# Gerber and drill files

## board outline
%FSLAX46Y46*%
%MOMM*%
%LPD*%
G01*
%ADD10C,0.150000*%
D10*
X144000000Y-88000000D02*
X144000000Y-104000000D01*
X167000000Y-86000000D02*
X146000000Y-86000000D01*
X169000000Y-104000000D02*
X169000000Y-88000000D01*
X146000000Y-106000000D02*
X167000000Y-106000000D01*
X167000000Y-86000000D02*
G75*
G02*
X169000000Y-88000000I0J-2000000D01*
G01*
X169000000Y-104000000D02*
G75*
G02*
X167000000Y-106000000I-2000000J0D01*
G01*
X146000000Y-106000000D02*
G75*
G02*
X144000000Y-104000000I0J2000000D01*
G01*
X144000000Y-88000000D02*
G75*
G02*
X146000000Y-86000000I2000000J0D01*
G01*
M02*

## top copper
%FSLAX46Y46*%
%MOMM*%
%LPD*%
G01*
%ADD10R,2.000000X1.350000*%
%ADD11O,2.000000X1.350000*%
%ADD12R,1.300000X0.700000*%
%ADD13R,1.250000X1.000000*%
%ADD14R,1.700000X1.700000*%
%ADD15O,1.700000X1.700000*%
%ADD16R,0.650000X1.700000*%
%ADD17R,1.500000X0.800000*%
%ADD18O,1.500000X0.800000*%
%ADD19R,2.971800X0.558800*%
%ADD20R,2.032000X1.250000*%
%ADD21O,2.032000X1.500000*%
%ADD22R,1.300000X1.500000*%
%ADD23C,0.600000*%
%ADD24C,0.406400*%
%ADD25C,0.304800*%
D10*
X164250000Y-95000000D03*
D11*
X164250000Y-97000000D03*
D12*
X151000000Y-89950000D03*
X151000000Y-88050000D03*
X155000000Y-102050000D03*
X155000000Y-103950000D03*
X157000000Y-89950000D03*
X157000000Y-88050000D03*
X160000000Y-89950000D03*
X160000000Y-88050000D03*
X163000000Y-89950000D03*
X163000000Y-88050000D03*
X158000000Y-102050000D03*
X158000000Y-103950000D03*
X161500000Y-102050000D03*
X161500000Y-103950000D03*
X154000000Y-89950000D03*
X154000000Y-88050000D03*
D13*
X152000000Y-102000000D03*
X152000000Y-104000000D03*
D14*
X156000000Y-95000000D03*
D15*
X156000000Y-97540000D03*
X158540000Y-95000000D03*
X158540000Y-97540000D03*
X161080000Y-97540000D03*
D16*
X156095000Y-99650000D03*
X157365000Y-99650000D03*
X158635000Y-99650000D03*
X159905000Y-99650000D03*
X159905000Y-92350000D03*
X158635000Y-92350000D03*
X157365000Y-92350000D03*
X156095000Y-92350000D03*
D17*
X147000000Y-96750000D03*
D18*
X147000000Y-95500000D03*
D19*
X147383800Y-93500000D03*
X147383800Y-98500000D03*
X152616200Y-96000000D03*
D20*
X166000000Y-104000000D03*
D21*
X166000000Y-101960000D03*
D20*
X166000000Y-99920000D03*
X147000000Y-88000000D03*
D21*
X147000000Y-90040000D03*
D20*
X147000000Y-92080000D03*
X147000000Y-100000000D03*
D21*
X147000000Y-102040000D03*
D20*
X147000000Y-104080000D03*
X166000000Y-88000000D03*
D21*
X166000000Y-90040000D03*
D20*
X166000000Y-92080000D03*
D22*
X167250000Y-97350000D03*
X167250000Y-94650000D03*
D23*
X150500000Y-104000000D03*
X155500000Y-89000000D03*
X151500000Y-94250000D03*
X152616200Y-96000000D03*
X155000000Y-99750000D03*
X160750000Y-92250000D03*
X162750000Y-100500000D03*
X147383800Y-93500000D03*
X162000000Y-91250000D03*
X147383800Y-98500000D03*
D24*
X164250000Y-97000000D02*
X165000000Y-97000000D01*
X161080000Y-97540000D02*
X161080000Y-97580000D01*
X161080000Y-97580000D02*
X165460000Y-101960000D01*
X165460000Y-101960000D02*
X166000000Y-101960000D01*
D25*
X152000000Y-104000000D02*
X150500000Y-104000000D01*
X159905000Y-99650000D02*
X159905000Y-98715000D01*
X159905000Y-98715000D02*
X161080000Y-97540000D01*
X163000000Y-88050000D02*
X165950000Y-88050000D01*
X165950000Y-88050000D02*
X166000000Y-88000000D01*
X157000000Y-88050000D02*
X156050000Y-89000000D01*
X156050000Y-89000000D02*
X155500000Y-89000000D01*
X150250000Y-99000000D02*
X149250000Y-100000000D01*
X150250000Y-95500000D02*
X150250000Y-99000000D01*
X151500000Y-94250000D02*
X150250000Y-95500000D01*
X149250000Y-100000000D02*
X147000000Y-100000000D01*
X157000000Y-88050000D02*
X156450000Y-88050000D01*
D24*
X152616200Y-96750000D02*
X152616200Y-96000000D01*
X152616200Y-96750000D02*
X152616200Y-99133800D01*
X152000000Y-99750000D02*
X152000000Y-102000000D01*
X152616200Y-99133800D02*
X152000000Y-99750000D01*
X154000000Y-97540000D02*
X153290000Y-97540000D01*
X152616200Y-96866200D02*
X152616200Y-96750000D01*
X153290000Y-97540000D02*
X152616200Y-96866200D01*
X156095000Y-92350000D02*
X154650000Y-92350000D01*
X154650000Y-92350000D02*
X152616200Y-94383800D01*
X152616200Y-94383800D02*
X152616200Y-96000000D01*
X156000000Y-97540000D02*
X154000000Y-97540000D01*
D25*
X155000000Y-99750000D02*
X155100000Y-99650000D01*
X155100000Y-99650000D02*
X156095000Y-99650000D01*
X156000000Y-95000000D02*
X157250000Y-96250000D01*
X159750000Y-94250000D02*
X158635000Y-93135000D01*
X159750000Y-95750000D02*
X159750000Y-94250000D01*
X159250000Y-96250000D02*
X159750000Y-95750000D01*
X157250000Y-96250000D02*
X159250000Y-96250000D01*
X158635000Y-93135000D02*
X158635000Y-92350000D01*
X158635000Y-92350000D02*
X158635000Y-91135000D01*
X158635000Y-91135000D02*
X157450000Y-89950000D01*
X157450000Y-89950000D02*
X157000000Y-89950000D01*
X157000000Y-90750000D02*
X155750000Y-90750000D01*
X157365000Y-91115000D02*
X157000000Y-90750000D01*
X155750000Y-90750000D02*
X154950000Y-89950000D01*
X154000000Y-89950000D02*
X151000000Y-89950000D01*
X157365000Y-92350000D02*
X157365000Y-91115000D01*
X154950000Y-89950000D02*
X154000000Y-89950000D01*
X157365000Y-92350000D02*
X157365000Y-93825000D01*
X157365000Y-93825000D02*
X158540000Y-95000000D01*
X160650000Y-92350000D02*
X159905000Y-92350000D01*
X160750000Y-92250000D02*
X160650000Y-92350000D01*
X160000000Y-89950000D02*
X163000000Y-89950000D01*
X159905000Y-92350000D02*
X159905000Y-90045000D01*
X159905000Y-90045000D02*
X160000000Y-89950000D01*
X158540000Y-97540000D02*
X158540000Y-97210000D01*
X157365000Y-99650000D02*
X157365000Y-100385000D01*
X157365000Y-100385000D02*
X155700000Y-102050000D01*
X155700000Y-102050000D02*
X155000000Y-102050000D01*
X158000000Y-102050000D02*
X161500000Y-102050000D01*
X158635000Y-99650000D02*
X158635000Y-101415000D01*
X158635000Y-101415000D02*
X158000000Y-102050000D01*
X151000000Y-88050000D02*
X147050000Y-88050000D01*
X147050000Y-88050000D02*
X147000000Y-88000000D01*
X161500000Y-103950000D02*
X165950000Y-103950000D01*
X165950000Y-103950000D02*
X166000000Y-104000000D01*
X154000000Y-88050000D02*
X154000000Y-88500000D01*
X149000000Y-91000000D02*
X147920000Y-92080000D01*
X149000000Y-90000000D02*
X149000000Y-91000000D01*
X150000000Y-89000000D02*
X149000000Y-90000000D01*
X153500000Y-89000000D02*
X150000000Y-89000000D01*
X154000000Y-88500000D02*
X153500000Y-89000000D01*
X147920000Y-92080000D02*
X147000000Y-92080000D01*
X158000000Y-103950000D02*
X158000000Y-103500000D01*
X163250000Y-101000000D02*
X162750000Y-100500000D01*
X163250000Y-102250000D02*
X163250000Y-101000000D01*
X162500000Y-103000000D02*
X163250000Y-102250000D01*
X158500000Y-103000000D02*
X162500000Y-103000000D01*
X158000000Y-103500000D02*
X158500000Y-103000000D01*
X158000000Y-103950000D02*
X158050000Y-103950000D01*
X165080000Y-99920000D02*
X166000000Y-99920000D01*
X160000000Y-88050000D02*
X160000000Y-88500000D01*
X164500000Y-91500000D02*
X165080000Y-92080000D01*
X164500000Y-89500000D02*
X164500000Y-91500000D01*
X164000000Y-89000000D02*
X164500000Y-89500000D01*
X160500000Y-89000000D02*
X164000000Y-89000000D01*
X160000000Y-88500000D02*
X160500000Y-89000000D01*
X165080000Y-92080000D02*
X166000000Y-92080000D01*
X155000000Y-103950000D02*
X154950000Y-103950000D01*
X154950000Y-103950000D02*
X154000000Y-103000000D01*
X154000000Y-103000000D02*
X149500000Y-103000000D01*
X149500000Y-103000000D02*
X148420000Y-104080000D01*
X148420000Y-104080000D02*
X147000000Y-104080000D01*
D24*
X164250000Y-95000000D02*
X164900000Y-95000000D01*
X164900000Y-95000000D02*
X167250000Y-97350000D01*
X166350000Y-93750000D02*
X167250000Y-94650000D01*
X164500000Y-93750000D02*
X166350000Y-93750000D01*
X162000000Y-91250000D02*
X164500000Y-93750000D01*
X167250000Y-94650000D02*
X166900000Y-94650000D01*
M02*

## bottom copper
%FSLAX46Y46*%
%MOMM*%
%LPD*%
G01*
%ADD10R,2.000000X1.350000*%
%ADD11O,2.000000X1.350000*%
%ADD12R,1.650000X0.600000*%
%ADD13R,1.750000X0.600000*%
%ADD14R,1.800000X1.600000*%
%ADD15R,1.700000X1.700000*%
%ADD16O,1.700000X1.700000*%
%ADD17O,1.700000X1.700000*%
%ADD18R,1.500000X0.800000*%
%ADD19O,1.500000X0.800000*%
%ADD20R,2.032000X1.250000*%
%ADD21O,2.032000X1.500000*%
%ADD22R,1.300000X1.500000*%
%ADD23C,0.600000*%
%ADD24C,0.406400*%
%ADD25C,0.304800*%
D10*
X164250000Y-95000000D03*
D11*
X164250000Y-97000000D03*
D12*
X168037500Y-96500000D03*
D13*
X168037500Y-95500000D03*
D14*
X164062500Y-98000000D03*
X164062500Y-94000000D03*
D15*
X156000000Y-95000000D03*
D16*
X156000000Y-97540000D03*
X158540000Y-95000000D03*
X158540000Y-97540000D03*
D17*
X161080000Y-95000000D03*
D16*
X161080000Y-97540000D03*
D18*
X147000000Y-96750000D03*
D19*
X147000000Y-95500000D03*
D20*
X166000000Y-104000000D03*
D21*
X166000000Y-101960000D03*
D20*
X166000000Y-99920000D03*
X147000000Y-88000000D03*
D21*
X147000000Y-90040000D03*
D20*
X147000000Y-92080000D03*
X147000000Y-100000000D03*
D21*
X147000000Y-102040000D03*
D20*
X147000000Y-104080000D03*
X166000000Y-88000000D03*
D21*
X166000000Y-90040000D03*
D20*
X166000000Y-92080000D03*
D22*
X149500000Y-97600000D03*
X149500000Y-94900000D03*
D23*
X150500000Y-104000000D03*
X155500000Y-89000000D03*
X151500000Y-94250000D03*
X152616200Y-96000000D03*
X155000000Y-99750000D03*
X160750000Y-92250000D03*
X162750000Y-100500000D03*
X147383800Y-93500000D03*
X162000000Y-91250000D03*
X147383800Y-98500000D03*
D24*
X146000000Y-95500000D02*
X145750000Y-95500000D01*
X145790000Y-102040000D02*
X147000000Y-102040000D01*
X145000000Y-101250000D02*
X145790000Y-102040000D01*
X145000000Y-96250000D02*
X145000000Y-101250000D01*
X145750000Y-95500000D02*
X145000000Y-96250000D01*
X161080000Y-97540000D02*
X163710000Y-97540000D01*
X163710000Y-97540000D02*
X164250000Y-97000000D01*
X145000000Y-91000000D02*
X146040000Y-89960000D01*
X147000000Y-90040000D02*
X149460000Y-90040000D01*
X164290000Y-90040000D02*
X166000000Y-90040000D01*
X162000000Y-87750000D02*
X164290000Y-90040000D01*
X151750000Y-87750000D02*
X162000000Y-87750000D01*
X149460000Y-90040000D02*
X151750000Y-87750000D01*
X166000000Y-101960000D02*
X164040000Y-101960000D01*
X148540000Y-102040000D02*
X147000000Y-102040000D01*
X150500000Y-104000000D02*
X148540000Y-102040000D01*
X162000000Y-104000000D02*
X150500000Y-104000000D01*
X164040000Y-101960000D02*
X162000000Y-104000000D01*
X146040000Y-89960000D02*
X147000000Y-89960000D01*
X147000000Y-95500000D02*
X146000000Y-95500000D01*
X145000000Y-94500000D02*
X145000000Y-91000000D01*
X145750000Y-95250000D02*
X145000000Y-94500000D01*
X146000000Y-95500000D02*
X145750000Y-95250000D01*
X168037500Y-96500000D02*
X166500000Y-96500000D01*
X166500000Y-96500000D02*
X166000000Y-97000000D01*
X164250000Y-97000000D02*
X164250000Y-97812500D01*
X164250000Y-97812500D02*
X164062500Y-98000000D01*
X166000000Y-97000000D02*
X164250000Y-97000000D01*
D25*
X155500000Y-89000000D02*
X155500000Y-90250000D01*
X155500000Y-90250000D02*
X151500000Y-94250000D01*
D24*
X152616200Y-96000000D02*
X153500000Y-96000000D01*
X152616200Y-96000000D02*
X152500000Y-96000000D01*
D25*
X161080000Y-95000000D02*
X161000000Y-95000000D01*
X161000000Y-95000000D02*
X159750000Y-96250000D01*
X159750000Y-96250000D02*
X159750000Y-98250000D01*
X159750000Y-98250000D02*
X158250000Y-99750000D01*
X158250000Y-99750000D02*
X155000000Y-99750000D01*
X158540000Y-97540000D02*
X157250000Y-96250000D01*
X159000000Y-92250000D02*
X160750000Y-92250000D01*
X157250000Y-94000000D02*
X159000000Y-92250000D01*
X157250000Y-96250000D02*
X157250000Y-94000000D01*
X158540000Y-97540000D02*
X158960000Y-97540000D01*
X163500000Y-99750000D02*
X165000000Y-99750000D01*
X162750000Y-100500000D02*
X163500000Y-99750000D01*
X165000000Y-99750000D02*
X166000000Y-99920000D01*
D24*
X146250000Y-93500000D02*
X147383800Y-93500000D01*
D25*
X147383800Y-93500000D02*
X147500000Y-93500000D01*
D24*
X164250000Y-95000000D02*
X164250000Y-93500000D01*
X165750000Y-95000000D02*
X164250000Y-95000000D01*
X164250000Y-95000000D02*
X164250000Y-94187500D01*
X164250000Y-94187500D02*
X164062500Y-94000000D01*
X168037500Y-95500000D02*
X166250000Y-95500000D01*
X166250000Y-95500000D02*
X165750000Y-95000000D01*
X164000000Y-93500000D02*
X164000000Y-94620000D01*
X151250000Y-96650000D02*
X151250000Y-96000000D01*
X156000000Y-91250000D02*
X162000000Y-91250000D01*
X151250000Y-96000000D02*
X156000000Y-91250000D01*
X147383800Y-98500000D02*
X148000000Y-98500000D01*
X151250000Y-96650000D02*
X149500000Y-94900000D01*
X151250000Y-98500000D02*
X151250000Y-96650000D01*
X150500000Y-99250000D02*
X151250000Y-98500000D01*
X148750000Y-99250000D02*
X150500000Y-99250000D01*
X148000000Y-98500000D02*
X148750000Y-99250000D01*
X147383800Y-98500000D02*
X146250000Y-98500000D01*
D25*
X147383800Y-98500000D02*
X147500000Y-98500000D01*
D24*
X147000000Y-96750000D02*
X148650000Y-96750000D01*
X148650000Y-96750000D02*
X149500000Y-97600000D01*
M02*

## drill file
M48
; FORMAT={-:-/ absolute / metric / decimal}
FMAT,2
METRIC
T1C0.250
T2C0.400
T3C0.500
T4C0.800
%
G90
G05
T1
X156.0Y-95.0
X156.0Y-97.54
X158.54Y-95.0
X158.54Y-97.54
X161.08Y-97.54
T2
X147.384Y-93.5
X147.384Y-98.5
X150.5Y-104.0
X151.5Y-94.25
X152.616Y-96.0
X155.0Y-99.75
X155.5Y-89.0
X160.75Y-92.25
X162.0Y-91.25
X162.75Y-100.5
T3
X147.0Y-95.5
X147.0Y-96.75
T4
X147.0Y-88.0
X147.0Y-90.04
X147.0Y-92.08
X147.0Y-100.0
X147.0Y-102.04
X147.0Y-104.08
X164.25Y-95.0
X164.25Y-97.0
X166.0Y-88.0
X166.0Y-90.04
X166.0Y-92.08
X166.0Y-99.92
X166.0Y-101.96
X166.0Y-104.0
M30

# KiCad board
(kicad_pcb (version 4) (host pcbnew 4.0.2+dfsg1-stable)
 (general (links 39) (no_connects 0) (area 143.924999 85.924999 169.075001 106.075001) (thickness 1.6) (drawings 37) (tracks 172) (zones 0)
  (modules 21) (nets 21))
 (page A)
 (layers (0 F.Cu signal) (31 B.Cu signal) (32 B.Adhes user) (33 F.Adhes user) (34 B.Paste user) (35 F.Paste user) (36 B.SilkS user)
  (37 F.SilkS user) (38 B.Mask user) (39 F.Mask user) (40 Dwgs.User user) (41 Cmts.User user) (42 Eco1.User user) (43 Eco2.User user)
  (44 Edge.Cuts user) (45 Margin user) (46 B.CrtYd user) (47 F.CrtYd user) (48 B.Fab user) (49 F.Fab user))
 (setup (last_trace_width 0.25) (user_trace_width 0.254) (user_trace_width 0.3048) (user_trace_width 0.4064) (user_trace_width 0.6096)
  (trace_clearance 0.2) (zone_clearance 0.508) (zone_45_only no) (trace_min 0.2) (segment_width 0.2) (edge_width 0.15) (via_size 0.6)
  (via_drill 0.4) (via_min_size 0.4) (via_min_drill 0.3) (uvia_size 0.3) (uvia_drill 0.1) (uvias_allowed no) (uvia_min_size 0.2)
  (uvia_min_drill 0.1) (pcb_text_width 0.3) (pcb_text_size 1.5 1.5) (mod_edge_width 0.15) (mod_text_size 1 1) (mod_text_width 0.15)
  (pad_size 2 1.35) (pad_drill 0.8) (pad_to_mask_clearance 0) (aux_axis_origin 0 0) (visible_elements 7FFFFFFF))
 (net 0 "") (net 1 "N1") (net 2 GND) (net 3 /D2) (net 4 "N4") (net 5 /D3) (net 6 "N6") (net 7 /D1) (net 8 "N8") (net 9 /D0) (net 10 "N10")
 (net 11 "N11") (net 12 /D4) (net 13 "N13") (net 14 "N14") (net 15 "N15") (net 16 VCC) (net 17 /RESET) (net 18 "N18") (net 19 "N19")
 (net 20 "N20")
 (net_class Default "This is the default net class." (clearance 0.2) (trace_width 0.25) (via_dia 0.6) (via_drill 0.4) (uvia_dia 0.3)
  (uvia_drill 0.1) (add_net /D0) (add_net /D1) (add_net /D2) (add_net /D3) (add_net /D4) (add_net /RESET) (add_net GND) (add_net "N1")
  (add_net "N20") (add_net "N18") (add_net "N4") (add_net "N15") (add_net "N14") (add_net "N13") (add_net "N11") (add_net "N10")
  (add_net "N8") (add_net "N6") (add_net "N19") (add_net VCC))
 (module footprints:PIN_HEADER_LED (layer B.Cu) (at 164.25 95 180)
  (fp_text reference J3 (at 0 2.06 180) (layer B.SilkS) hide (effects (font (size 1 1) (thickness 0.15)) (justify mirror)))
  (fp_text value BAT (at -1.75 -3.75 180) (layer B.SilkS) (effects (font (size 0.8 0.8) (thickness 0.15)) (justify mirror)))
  (pad 1 thru_hole rect (at 0 0 180) (size 2 1.35) (drill 0.8) (layers *.Cu *.Mask) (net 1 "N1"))
  (pad 2 thru_hole oval (at 0 -2 180) (size 2 1.35) (drill 0.8) (layers *.Cu *.Mask) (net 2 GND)))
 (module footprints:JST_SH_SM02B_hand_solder (layer B.Cu) (at 166 96 90)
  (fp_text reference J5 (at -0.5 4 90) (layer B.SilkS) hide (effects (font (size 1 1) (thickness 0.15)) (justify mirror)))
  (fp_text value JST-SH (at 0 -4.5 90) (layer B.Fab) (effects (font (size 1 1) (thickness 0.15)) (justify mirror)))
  (pad 1 smd rect (at -0.5 2.0375 90) (size 0.6 1.65) (layers B.Cu B.Paste B.Mask) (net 2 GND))
  (pad 2 smd rect (at 0.5 2.0375 90) (size 0.6 1.75) (layers B.Cu B.Paste B.Mask) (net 1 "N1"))
  (pad 1 smd rect (at -2 -1.9375 90) (size 1.6 1.8) (layers B.Cu B.Paste B.Mask) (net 2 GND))
  (pad 2 smd rect (at 2 -1.9375 90) (size 1.6 1.8) (layers B.Cu B.Paste B.Mask) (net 1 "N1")))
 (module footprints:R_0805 (layer F.Cu) (at 151 89 90)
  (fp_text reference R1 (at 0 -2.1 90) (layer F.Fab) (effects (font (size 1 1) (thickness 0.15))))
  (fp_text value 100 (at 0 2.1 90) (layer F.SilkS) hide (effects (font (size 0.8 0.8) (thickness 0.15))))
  (pad 1 smd rect (at -0.95 0 90) (size 0.7 1.3) (layers F.Cu F.Paste F.Mask) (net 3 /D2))
  (pad 2 smd rect (at 0.95 0 90) (size 0.7 1.3) (layers F.Cu F.Paste F.Mask) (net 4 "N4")))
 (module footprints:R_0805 (layer F.Cu) (at 155 103 270)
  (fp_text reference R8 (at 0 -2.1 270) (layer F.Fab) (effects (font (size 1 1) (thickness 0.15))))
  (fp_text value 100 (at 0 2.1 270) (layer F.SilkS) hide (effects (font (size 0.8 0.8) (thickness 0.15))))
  (pad 1 smd rect (at -0.95 0 270) (size 0.7 1.3) (layers F.Cu F.Paste F.Mask) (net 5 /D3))
  (pad 2 smd rect (at 0.95 0 270) (size 0.7 1.3) (layers F.Cu F.Paste F.Mask) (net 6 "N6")))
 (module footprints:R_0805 (layer F.Cu) (at 157 89 90)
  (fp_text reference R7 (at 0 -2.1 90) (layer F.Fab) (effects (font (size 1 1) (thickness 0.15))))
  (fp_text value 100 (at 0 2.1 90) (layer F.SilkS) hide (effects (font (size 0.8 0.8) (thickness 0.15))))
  (pad 1 smd rect (at -0.95 0 90) (size 0.7 1.3) (layers F.Cu F.Paste F.Mask) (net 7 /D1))
  (pad 2 smd rect (at 0.95 0 90) (size 0.7 1.3) (layers F.Cu F.Paste F.Mask) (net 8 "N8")))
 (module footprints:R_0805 (layer F.Cu) (at 160 89 90)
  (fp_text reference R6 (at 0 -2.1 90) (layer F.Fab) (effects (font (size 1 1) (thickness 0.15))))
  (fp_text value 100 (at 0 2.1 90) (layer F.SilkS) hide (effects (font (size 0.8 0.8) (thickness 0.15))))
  (pad 1 smd rect (at -0.95 0 90) (size 0.7 1.3) (layers F.Cu F.Paste F.Mask) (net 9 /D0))
  (pad 2 smd rect (at 0.95 0 90) (size 0.7 1.3) (layers F.Cu F.Paste F.Mask) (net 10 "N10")))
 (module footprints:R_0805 (layer F.Cu) (at 163 89 90)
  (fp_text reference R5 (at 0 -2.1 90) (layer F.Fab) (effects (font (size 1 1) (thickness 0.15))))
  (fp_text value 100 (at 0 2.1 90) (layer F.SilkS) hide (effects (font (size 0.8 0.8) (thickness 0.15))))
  (pad 1 smd rect (at -0.95 0 90) (size 0.7 1.3) (layers F.Cu F.Paste F.Mask) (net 9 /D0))
  (pad 2 smd rect (at 0.95 0 90) (size 0.7 1.3) (layers F.Cu F.Paste F.Mask) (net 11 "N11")))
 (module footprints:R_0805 (layer F.Cu) (at 158 103 270)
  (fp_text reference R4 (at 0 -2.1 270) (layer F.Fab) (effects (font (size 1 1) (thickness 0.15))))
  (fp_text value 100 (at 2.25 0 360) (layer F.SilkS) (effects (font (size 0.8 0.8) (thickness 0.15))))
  (pad 1 smd rect (at -0.95 0 270) (size 0.7 1.3) (layers F.Cu F.Paste F.Mask) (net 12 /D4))
  (pad 2 smd rect (at 0.95 0 270) (size 0.7 1.3) (layers F.Cu F.Paste F.Mask) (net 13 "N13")))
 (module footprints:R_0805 (layer F.Cu) (at 161.5 103 270)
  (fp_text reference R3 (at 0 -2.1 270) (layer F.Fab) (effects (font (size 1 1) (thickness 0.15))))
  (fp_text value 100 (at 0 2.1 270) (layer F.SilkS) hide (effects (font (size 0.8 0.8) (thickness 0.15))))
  (pad 1 smd rect (at -0.95 0 270) (size 0.7 1.3) (layers F.Cu F.Paste F.Mask) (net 12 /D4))
  (pad 2 smd rect (at 0.95 0 270) (size 0.7 1.3) (layers F.Cu F.Paste F.Mask) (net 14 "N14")))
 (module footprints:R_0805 (layer F.Cu) (at 154 89 90)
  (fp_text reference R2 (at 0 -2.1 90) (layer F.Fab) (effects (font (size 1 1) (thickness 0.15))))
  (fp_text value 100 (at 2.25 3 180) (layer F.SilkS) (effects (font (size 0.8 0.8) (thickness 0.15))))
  (pad 1 smd rect (at -0.95 0 90) (size 0.7 1.3) (layers F.Cu F.Paste F.Mask) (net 3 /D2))
  (pad 2 smd rect (at 0.95 0 90) (size 0.7 1.3) (layers F.Cu F.Paste F.Mask) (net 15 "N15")))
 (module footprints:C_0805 (layer F.Cu) (at 152 103 270)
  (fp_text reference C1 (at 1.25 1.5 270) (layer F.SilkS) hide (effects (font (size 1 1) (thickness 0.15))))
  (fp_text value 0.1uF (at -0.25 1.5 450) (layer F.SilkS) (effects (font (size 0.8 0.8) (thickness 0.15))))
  (pad 1 smd rect (at -1 0 270) (size 1 1.25) (layers F.Cu F.Paste F.Mask) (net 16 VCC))
  (pad 2 smd rect (at 1 0 270) (size 1 1.25) (layers F.Cu F.Paste F.Mask) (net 2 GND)))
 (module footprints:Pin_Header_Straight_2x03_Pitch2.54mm (layer B.Cu) (at 156 95 270)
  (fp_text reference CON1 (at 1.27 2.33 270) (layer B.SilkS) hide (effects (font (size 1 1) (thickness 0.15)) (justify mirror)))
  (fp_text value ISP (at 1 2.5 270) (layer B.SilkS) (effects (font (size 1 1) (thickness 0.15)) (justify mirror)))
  (pad 1 thru_hole rect (at 0 0 270) (size 1.7 1.7) (drill 0.25) (layers *.Cu B.SilkS B.Mask) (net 7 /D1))
  (pad 2 thru_hole oval (at 2.54 0 270) (size 1.7 1.7) (drill 0.25) (layers *.Cu B.SilkS B.Mask) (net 16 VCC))
  (pad 3 thru_hole oval (at 0 -2.54 270) (size 1.7 1.7) (drill 0.25) (layers *.Cu B.SilkS B.Mask) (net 3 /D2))
  (pad 4 thru_hole oval (at 2.54 -2.54 270) (size 1.7 1.7) (drill 0.25) (layers *.Cu B.SilkS B.Mask) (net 9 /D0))
  (pad 5 smd oval (at 0 -5.08 270) (size 1.7 1.7) (layers B.Cu B.Paste B.Mask) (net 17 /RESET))
  (pad 6 thru_hole oval (at 2.54 -5.08 270) (size 1.7 1.7) (drill 0.25) (layers *.Cu B.SilkS B.Mask) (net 2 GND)))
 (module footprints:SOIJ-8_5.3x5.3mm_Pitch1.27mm (layer F.Cu) (at 158 96 90)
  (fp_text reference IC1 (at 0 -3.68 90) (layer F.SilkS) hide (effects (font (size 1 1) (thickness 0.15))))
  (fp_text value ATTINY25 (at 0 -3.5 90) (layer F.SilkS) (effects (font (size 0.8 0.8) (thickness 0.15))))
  (pad 1 smd rect (at -3.65 -1.905 90) (size 1.7 0.65) (layers F.Cu F.Paste F.Mask) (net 17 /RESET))
  (pad 2 smd rect (at -3.65 -0.635 90) (size 1.7 0.65) (layers F.Cu F.Paste F.Mask) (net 5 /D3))
  (pad 3 smd rect (at -3.65 0.635 90) (size 1.7 0.65) (layers F.Cu F.Paste F.Mask) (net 12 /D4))
  (pad 4 smd rect (at -3.65 1.905 90) (size 1.7 0.65) (layers F.Cu F.Paste F.Mask) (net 2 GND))
  (pad 5 smd rect (at 3.65 1.905 90) (size 1.7 0.65) (layers F.Cu F.Paste F.Mask) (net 9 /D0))
  (pad 6 smd rect (at 3.65 0.635 90) (size 1.7 0.65) (layers F.Cu F.Paste F.Mask) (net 7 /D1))
  (pad 7 smd rect (at 3.65 -0.635 90) (size 1.7 0.65) (layers F.Cu F.Paste F.Mask) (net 3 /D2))
  (pad 8 smd rect (at 3.65 -1.905 90) (size 1.7 0.65) (layers F.Cu F.Paste F.Mask) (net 16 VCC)))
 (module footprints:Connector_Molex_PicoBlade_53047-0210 (layer F.Cu) (at 147 96.75 90)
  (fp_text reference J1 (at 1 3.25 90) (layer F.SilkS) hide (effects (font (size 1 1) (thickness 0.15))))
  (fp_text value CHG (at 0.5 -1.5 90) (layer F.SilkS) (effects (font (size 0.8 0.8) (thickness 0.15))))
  (pad 1 thru_hole rect (at 0 0 90) (size 0.8 1.5) (drill 0.5) (layers *.Cu *.Mask F.SilkS) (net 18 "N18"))
  (pad 2 thru_hole oval (at 1.25 0 90) (size 0.8 1.5) (drill 0.5) (layers *.Cu *.Mask F.SilkS) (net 2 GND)))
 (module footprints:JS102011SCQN (layer F.Cu) (at 150 96)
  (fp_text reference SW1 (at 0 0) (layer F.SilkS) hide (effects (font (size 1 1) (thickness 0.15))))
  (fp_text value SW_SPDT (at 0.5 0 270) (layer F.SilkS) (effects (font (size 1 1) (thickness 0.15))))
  (pad 1 smd rect (at -2.6162 -2.5) (size 2.9718 0.5588) (layers F.Cu F.Paste F.Mask) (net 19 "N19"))
  (pad 3 smd rect (at -2.6162 2.5) (size 2.9718 0.5588) (layers F.Cu F.Paste F.Mask) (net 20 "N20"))
  (pad 2 smd rect (at 2.6162 0) (size 2.9718 0.5588) (layers F.Cu F.Paste F.Mask) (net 16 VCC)))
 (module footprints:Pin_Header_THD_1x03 (layer F.Cu) (at 166 104 180)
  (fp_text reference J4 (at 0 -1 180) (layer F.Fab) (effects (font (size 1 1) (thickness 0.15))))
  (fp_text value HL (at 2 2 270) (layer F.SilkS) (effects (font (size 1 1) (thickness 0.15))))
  (pad 1 thru_hole rect (at 0 0 180) (size 2.032 1.25) (drill 0.8) (layers *.Cu *.Mask F.SilkS) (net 14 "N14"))
  (pad 2 thru_hole oval (at 0 2.04 180) (size 2.032 1.5) (drill 0.8) (layers *.Cu *.Mask F.SilkS) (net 2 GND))
  (pad 3 thru_hole rect (at 0 4.08 180) (size 2.032 1.25) (drill 0.8) (layers *.Cu *.Mask F.SilkS) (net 13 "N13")))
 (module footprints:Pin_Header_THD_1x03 (layer F.Cu) (at 147 88)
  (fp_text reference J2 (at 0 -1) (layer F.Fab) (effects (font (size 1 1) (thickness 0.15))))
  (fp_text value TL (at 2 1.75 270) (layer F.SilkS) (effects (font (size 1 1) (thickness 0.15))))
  (pad 1 thru_hole rect (at 0 0) (size 2.032 1.25) (drill 0.8) (layers *.Cu *.Mask F.SilkS) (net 4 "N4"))
  (pad 2 thru_hole oval (at 0 2.04) (size 2.032 1.5) (drill 0.8) (layers *.Cu *.Mask F.SilkS) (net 2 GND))
  (pad 3 thru_hole rect (at 0 4.08) (size 2.032 1.25) (drill 0.8) (layers *.Cu *.Mask F.SilkS) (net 15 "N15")))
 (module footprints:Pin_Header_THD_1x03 (layer F.Cu) (at 147 100)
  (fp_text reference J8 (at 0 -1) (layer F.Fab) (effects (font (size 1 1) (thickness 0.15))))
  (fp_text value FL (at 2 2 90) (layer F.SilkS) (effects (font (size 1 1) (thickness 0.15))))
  (pad 1 thru_hole rect (at 0 0) (size 2.032 1.25) (drill 0.8) (layers *.Cu *.Mask F.SilkS) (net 8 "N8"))
  (pad 2 thru_hole oval (at 0 2.04) (size 2.032 1.5) (drill 0.8) (layers *.Cu *.Mask F.SilkS) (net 2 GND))
  (pad 3 thru_hole rect (at 0 4.08) (size 2.032 1.25) (drill 0.8) (layers *.Cu *.Mask F.SilkS) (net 6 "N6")))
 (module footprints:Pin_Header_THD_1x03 (layer F.Cu) (at 166 88)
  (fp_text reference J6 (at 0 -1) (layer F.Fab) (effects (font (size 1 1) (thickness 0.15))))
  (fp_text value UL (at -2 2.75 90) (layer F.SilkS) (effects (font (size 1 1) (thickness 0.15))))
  (pad 1 thru_hole rect (at 0 0) (size 2.032 1.25) (drill 0.8) (layers *.Cu *.Mask F.SilkS) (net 11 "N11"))
  (pad 2 thru_hole oval (at 0 2.04) (size 2.032 1.5) (drill 0.8) (layers *.Cu *.Mask F.SilkS) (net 2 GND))
  (pad 3 thru_hole rect (at 0 4.08) (size 2.032 1.25) (drill 0.8) (layers *.Cu *.Mask F.SilkS) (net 10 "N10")))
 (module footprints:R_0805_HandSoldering (layer F.Cu) (at 167.25 96 90)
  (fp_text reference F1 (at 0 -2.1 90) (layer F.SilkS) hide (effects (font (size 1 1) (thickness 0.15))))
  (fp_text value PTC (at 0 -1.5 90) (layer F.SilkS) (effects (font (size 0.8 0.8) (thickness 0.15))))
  (pad 1 smd rect (at -1.35 0 90) (size 1.5 1.3) (layers F.Cu F.Paste F.Mask) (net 1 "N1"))
  (pad 2 smd rect (at 1.35 0 90) (size 1.5 1.3) (layers F.Cu F.Paste F.Mask) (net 20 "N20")))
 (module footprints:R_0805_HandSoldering (layer B.Cu) (at 149.5 96.25 90)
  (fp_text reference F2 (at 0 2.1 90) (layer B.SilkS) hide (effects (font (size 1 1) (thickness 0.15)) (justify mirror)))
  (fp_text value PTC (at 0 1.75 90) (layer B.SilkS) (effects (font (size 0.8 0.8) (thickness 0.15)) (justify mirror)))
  (pad 1 smd rect (at -1.35 0 90) (size 1.5 1.3) (layers B.Cu B.Paste B.Mask) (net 18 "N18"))
  (pad 2 smd rect (at 1.35 0 90) (size 1.5 1.3) (layers B.Cu B.Paste B.Mask) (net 20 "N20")))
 (gr_line (start 144 88) (end 144 104) (angle 90) (layer Edge.Cuts) (width 0.15))
 (gr_line (start 167 86) (end 146 86) (angle 90) (layer Edge.Cuts) (width 0.15))
 (gr_line (start 169 104) (end 169 88) (angle 90) (layer Edge.Cuts) (width 0.15))
 (gr_line (start 146 106) (end 167 106) (angle 90) (layer Edge.Cuts) (width 0.15))
 (gr_arc (start 167 88) (end 167 86) (angle 90) (layer Edge.Cuts) (width 0.15))
 (gr_arc (start 167 104) (end 169 104) (angle 90) (layer Edge.Cuts) (width 0.15))
 (gr_arc (start 146 104) (end 146 106) (angle 90) (layer Edge.Cuts) (width 0.15))
 (gr_arc (start 146 88) (end 144 88) (angle 90) (layer Edge.Cuts) (width 0.15))
 (segment (start 146 95.5) (end 145.75 95.5) (width 0.4064) (layer B.Cu) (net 2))
 (segment (start 145.79 102.04) (end 147 102.04) (width 0.4064) (layer B.Cu) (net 2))
 (segment (start 145 101.25) (end 145.79 102.04) (width 0.4064) (layer B.Cu) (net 2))
 (segment (start 145 96.25) (end 145 101.25) (width 0.4064) (layer B.Cu) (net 2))
 (segment (start 145.75 95.5) (end 145 96.25) (width 0.4064) (layer B.Cu) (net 2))
 (segment (start 164.25 97) (end 165 97) (width 0.4064) (layer F.Cu) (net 2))
 (segment (start 161.08 97.54) (end 163.71 97.54) (width 0.4064) (layer B.Cu) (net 2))
 (segment (start 163.71 97.54) (end 164.25 97) (width 0.4064) (layer B.Cu) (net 2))
 (segment (start 145 91) (end 146.04 89.96) (width 0.4064) (layer B.Cu) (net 2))
 (segment (start 161.08 97.54) (end 161.08 97.58) (width 0.4064) (layer F.Cu) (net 2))
 (segment (start 161.08 97.58) (end 165.46 101.96) (width 0.4064) (layer F.Cu) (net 2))
 (segment (start 165.46 101.96) (end 166 101.96) (width 0.4064) (layer F.Cu) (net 2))
 (segment (start 147 90.04) (end 149.46 90.04) (width 0.4064) (layer B.Cu) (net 2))
 (segment (start 164.29 90.04) (end 166 90.04) (width 0.4064) (layer B.Cu) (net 2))
 (segment (start 162 87.75) (end 164.29 90.04) (width 0.4064) (layer B.Cu) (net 2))
 (segment (start 151.75 87.75) (end 162 87.75) (width 0.4064) (layer B.Cu) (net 2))
 (segment (start 149.46 90.04) (end 151.75 87.75) (width 0.4064) (layer B.Cu) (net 2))
 (segment (start 152 104) (end 150.5 104) (width 0.3048) (layer F.Cu) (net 2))
 (via (at 150.5 104) (size 0.6) (drill 0.4) (layers F.Cu B.Cu) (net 2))
 (segment (start 166 101.96) (end 164.04 101.96) (width 0.4064) (layer B.Cu) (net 2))
 (segment (start 148.54 102.04) (end 147 102.04) (width 0.4064) (layer B.Cu) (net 2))
 (segment (start 150.5 104) (end 148.54 102.04) (width 0.4064) (layer B.Cu) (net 2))
 (segment (start 162 104) (end 150.5 104) (width 0.4064) (layer B.Cu) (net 2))
 (segment (start 164.04 101.96) (end 162 104) (width 0.4064) (layer B.Cu) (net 2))
 (segment (start 146.04 89.96) (end 147 89.96) (width 0.4064) (layer B.Cu) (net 2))
 (segment (start 159.905 99.65) (end 159.905 98.715) (width 0.3048) (layer F.Cu) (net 2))
 (segment (start 159.905 98.715) (end 161.08 97.54) (width 0.3048) (layer F.Cu) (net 2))
 (segment (start 147 95.5) (end 146 95.5) (width 0.4064) (layer B.Cu) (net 2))
 (segment (start 145 94.5) (end 145 91) (width 0.4064) (layer B.Cu) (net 2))
 (segment (start 145.75 95.25) (end 145 94.5) (width 0.4064) (layer B.Cu) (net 2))
 (segment (start 146 95.5) (end 145.75 95.25) (width 0.4064) (layer B.Cu) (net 2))
 (segment (start 168.0375 96.5) (end 166.5 96.5) (width 0.4064) (layer B.Cu) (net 2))
 (segment (start 166.5 96.5) (end 166 97) (width 0.4064) (layer B.Cu) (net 2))
 (segment (start 164.25 97) (end 164.25 97.8125) (width 0.4064) (layer B.Cu) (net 2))
 (segment (start 164.25 97.8125) (end 164.0625 98) (width 0.4064) (layer B.Cu) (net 2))
 (segment (start 166 97) (end 164.25 97) (width 0.4064) (layer B.Cu) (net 2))
 (segment (start 163 88.05) (end 165.95 88.05) (width 0.3048) (layer F.Cu) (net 11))
 (segment (start 165.95 88.05) (end 166 88) (width 0.3048) (layer F.Cu) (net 11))
 (segment (start 155.5 89) (end 155.5 90.25) (width 0.3048) (layer B.Cu) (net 8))
 (segment (start 157 88.05) (end 156.05 89) (width 0.3048) (layer F.Cu) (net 8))
 (segment (start 156.05 89) (end 155.5 89) (width 0.3048) (layer F.Cu) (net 8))
 (via (at 155.5 89) (size 0.6) (drill 0.4) (layers F.Cu B.Cu) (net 8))
 (segment (start 150.25 99) (end 149.25 100) (width 0.3048) (layer F.Cu) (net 8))
 (segment (start 150.25 95.5) (end 150.25 99) (width 0.3048) (layer F.Cu) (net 8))
 (segment (start 151.5 94.25) (end 150.25 95.5) (width 0.3048) (layer F.Cu) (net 8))
 (via (at 151.5 94.25) (size 0.6) (drill 0.4) (layers F.Cu B.Cu) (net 8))
 (segment (start 155.5 90.25) (end 151.5 94.25) (width 0.3048) (layer B.Cu) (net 8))
 (segment (start 149.25 100) (end 147 100) (width 0.3048) (layer F.Cu) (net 8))
 (segment (start 157 88.05) (end 156.45 88.05) (width 0.3048) (layer F.Cu) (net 8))
 (segment (start 152.6162 96) (end 153.5 96) (width 0.4064) (layer B.Cu) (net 16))
 (segment (start 152.6162 96.75) (end 152.6162 96) (width 0.4064) (layer F.Cu) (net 16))
 (via (at 152.6162 96) (size 0.6) (drill 0.4) (layers F.Cu B.Cu) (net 16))
 (segment (start 152.6162 96) (end 152.5 96) (width 0.4064) (layer B.Cu) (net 16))
 (segment (start 152.6162 96.75) (end 152.6162 99.1338) (width 0.4064) (layer F.Cu) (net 16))
 (segment (start 152 99.75) (end 152 102) (width 0.4064) (layer F.Cu) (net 16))
 (segment (start 152.6162 99.1338) (end 152 99.75) (width 0.4064) (layer F.Cu) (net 16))
 (segment (start 154 97.54) (end 153.29 97.54) (width 0.4064) (layer F.Cu) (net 16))
 (segment (start 152.6162 96.8662) (end 152.6162 96.75) (width 0.4064) (layer F.Cu) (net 16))
 (segment (start 153.29 97.54) (end 152.6162 96.8662) (width 0.4064) (layer F.Cu) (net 16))
 (segment (start 156.095 92.35) (end 154.65 92.35) (width 0.4064) (layer F.Cu) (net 16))
 (segment (start 154.65 92.35) (end 152.6162 94.3838) (width 0.4064) (layer F.Cu) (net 16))
 (segment (start 152.6162 94.3838) (end 152.6162 96) (width 0.4064) (layer F.Cu) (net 16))
 (segment (start 156 97.54) (end 154 97.54) (width 0.4064) (layer F.Cu) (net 16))
 (segment (start 161.08 95) (end 161 95) (width 0.3048) (layer B.Cu) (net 17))
 (segment (start 161 95) (end 159.75 96.25) (width 0.3048) (layer B.Cu) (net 17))
 (segment (start 159.75 96.25) (end 159.75 98.25) (width 0.3048) (layer B.Cu) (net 17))
 (segment (start 159.75 98.25) (end 158.25 99.75) (width 0.3048) (layer B.Cu) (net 17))
 (segment (start 158.25 99.75) (end 155 99.75) (width 0.3048) (layer B.Cu) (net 17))
 (via (at 155 99.75) (size 0.6) (drill 0.4) (layers F.Cu B.Cu) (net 17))
 (segment (start 155 99.75) (end 155.1 99.65) (width 0.3048) (layer F.Cu) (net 17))
 (segment (start 155.1 99.65) (end 156.095 99.65) (width 0.3048) (layer F.Cu) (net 17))
 (segment (start 156 95) (end 157.25 96.25) (width 0.3048) (layer F.Cu) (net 7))
 (segment (start 159.75 94.25) (end 158.635 93.135) (width 0.3048) (layer F.Cu) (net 7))
 (segment (start 159.75 95.75) (end 159.75 94.25) (width 0.3048) (layer F.Cu) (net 7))
 (segment (start 159.25 96.25) (end 159.75 95.75) (width 0.3048) (layer F.Cu) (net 7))
 (segment (start 157.25 96.25) (end 159.25 96.25) (width 0.3048) (layer F.Cu) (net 7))
 (segment (start 158.635 93.135) (end 158.635 92.35) (width 0.3048) (layer F.Cu) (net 7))
 (segment (start 158.635 92.35) (end 158.635 91.135) (width 0.3048) (layer F.Cu) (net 7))
 (segment (start 158.635 91.135) (end 157.45 89.95) (width 0.3048) (layer F.Cu) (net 7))
 (segment (start 157.45 89.95) (end 157 89.95) (width 0.3048) (layer F.Cu) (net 7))
 (segment (start 157 90.75) (end 155.75 90.75) (width 0.3048) (layer F.Cu) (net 3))
 (segment (start 157.365 91.115) (end 157 90.75) (width 0.3048) (layer F.Cu) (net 3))
 (segment (start 155.75 90.75) (end 154.95 89.95) (width 0.3048) (layer F.Cu) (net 3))
 (segment (start 154 89.95) (end 151 89.95) (width 0.3048) (layer F.Cu) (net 3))
 (segment (start 157.365 92.35) (end 157.365 91.115) (width 0.3048) (layer F.Cu) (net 3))
 (segment (start 154.95 89.95) (end 154 89.95) (width 0.3048) (layer F.Cu) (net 3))
 (segment (start 157.365 92.35) (end 157.365 93.825) (width 0.3048) (layer F.Cu) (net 3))
 (segment (start 157.365 93.825) (end 158.54 95) (width 0.3048) (layer F.Cu) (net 3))
 (segment (start 158.54 97.54) (end 157.25 96.25) (width 0.3048) (layer B.Cu) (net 9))
 (segment (start 159 92.25) (end 160.75 92.25) (width 0.3048) (layer B.Cu) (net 9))
 (segment (start 157.25 94) (end 159 92.25) (width 0.3048) (layer B.Cu) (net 9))
 (segment (start 157.25 96.25) (end 157.25 94) (width 0.3048) (layer B.Cu) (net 9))
 (segment (start 158.54 97.54) (end 158.96 97.54) (width 0.3048) (layer B.Cu) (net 9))
 (segment (start 160.65 92.35) (end 159.905 92.35) (width 0.3048) (layer F.Cu) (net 9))
 (via (at 160.75 92.25) (size 0.6) (drill 0.4) (layers F.Cu B.Cu) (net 9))
 (segment (start 160.75 92.25) (end 160.65 92.35) (width 0.3048) (layer F.Cu) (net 9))
 (segment (start 160 89.95) (end 163 89.95) (width 0.3048) (layer F.Cu) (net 9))
 (segment (start 159.905 92.35) (end 159.905 90.045) (width 0.3048) (layer F.Cu) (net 9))
 (segment (start 159.905 90.045) (end 160 89.95) (width 0.3048) (layer F.Cu) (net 9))
 (segment (start 158.54 97.54) (end 158.54 97.21) (width 0.3048) (layer F.Cu) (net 9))
 (segment (start 157.365 99.65) (end 157.365 100.385) (width 0.3048) (layer F.Cu) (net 5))
 (segment (start 157.365 100.385) (end 155.7 102.05) (width 0.3048) (layer F.Cu) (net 5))
 (segment (start 155.7 102.05) (end 155 102.05) (width 0.3048) (layer F.Cu) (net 5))
 (segment (start 158 102.05) (end 161.5 102.05) (width 0.3048) (layer F.Cu) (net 12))
 (segment (start 158.635 99.65) (end 158.635 101.415) (width 0.3048) (layer F.Cu) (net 12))
 (segment (start 158.635 101.415) (end 158 102.05) (width 0.3048) (layer F.Cu) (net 12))
 (segment (start 151 88.05) (end 147.05 88.05) (width 0.3048) (layer F.Cu) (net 4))
 (segment (start 147.05 88.05) (end 147 88) (width 0.3048) (layer F.Cu) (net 4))
 (segment (start 161.5 103.95) (end 165.95 103.95) (width 0.3048) (layer F.Cu) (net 14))
 (segment (start 165.95 103.95) (end 166 104) (width 0.3048) (layer F.Cu) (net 14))
 (segment (start 154 88.05) (end 154 88.5) (width 0.3048) (layer F.Cu) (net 15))
 (segment (start 149 91) (end 147.92 92.08) (width 0.3048) (layer F.Cu) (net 15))
 (segment (start 149 90) (end 149 91) (width 0.3048) (layer F.Cu) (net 15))
 (segment (start 150 89) (end 149 90) (width 0.3048) (layer F.Cu) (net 15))
 (segment (start 153.5 89) (end 150 89) (width 0.3048) (layer F.Cu) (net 15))
 (segment (start 154 88.5) (end 153.5 89) (width 0.3048) (layer F.Cu) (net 15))
 (segment (start 147.92 92.08) (end 147 92.08) (width 0.3048) (layer F.Cu) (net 15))
 (segment (start 158 103.95) (end 158 103.5) (width 0.3048) (layer F.Cu) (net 13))
 (segment (start 163.5 99.75) (end 165 99.75) (width 0.3048) (layer B.Cu) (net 13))
 (segment (start 162.75 100.5) (end 163.5 99.75) (width 0.3048) (layer B.Cu) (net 13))
 (via (at 162.75 100.5) (size 0.6) (drill 0.4) (layers F.Cu B.Cu) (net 13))
 (segment (start 163.25 101) (end 162.75 100.5) (width 0.3048) (layer F.Cu) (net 13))
 (segment (start 163.25 102.25) (end 163.25 101) (width 0.3048) (layer F.Cu) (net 13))
 (segment (start 162.5 103) (end 163.25 102.25) (width 0.3048) (layer F.Cu) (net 13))
 (segment (start 158.5 103) (end 162.5 103) (width 0.3048) (layer F.Cu) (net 13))
 (segment (start 158 103.5) (end 158.5 103) (width 0.3048) (layer F.Cu) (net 13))
 (segment (start 165 99.75) (end 166 99.92) (width 0.3048) (layer B.Cu) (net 13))
 (segment (start 158 103.95) (end 158.05 103.95) (width 0.3048) (layer F.Cu) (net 13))
 (segment (start 165.08 99.92) (end 166 99.92) (width 0.3048) (layer F.Cu) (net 13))
 (segment (start 160 88.05) (end 160 88.5) (width 0.3048) (layer F.Cu) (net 10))
 (segment (start 164.5 91.5) (end 165.08 92.08) (width 0.3048) (layer F.Cu) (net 10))
 (segment (start 164.5 89.5) (end 164.5 91.5) (width 0.3048) (layer F.Cu) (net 10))
 (segment (start 164 89) (end 164.5 89.5) (width 0.3048) (layer F.Cu) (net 10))
 (segment (start 160.5 89) (end 164 89) (width 0.3048) (layer F.Cu) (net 10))
 (segment (start 160 88.5) (end 160.5 89) (width 0.3048) (layer F.Cu) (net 10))
 (segment (start 165.08 92.08) (end 166 92.08) (width 0.3048) (layer F.Cu) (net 10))
 (segment (start 155 103.95) (end 154.95 103.95) (width 0.3048) (layer F.Cu) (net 6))
 (segment (start 154.95 103.95) (end 154 103) (width 0.3048) (layer F.Cu) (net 6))
 (segment (start 154 103) (end 149.5 103) (width 0.3048) (layer F.Cu) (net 6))
 (segment (start 149.5 103) (end 148.42 104.08) (width 0.3048) (layer F.Cu) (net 6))
 (segment (start 148.42 104.08) (end 147 104.08) (width 0.3048) (layer F.Cu) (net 6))
 (segment (start 146.25 93.5) (end 147.3838 93.5) (width 0.4064) (layer B.Cu) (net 19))
 (segment (start 147.3838 93.5) (end 147.5 93.5) (width 0.3048) (layer B.Cu) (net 19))
 (via (at 147.3838 93.5) (size 0.6) (drill 0.4) (layers F.Cu B.Cu) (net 19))
 (segment (start 164.25 95) (end 164.9 95) (width 0.4064) (layer F.Cu) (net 1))
 (segment (start 164.9 95) (end 167.25 97.35) (width 0.4064) (layer F.Cu) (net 1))
 (segment (start 164.25 95) (end 164.25 93.5) (width 0.4064) (layer B.Cu) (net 1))
 (segment (start 165.75 95) (end 164.25 95) (width 0.4064) (layer B.Cu) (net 1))
 (segment (start 164.25 95) (end 164.25 94.1875) (width 0.4064) (layer B.Cu) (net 1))
 (segment (start 164.25 94.1875) (end 164.0625 94) (width 0.4064) (layer B.Cu) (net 1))
 (segment (start 168.0375 95.5) (end 166.25 95.5) (width 0.4064) (layer B.Cu) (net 1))
 (segment (start 166.25 95.5) (end 165.75 95) (width 0.4064) (layer B.Cu) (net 1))
 (segment (start 164 93.5) (end 164 94.62) (width 0.4064) (layer B.Cu) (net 1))
 (segment (start 151.25 96.65) (end 151.25 96) (width 0.4064) (layer B.Cu) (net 20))
 (segment (start 166.35 93.75) (end 167.25 94.65) (width 0.4064) (layer F.Cu) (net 20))
 (segment (start 164.5 93.75) (end 166.35 93.75) (width 0.4064) (layer F.Cu) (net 20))
 (segment (start 162 91.25) (end 164.5 93.75) (width 0.4064) (layer F.Cu) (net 20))
 (via (at 162 91.25) (size 0.6) (drill 0.4) (layers F.Cu B.Cu) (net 20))
 (segment (start 156 91.25) (end 162 91.25) (width 0.4064) (layer B.Cu) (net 20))
 (segment (start 151.25 96) (end 156 91.25) (width 0.4064) (layer B.Cu) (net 20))
 (segment (start 147.3838 98.5) (end 148 98.5) (width 0.4064) (layer B.Cu) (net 20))
 (via (at 147.3838 98.5) (size 0.6) (drill 0.4) (layers F.Cu B.Cu) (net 20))
 (segment (start 151.25 96.65) (end 149.5 94.9) (width 0.4064) (layer B.Cu) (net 20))
 (segment (start 151.25 98.5) (end 151.25 96.65) (width 0.4064) (layer B.Cu) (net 20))
 (segment (start 150.5 99.25) (end 151.25 98.5) (width 0.4064) (layer B.Cu) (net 20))
 (segment (start 148.75 99.25) (end 150.5 99.25) (width 0.4064) (layer B.Cu) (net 20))
 (segment (start 148 98.5) (end 148.75 99.25) (width 0.4064) (layer B.Cu) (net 20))
 (segment (start 167.25 94.65) (end 166.9 94.65) (width 0.4064) (layer F.Cu) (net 20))
 (segment (start 147.3838 98.5) (end 146.25 98.5) (width 0.4064) (layer B.Cu) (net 20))
 (segment (start 147.3838 98.5) (end 147.5 98.5) (width 0.3048) (layer B.Cu) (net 20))
 (segment (start 147 96.75) (end 148.65 96.75) (width 0.4064) (layer B.Cu) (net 18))
 (segment (start 148.65 96.75) (end 149.5 97.6) (width 0.4064) (layer B.Cu) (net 18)))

